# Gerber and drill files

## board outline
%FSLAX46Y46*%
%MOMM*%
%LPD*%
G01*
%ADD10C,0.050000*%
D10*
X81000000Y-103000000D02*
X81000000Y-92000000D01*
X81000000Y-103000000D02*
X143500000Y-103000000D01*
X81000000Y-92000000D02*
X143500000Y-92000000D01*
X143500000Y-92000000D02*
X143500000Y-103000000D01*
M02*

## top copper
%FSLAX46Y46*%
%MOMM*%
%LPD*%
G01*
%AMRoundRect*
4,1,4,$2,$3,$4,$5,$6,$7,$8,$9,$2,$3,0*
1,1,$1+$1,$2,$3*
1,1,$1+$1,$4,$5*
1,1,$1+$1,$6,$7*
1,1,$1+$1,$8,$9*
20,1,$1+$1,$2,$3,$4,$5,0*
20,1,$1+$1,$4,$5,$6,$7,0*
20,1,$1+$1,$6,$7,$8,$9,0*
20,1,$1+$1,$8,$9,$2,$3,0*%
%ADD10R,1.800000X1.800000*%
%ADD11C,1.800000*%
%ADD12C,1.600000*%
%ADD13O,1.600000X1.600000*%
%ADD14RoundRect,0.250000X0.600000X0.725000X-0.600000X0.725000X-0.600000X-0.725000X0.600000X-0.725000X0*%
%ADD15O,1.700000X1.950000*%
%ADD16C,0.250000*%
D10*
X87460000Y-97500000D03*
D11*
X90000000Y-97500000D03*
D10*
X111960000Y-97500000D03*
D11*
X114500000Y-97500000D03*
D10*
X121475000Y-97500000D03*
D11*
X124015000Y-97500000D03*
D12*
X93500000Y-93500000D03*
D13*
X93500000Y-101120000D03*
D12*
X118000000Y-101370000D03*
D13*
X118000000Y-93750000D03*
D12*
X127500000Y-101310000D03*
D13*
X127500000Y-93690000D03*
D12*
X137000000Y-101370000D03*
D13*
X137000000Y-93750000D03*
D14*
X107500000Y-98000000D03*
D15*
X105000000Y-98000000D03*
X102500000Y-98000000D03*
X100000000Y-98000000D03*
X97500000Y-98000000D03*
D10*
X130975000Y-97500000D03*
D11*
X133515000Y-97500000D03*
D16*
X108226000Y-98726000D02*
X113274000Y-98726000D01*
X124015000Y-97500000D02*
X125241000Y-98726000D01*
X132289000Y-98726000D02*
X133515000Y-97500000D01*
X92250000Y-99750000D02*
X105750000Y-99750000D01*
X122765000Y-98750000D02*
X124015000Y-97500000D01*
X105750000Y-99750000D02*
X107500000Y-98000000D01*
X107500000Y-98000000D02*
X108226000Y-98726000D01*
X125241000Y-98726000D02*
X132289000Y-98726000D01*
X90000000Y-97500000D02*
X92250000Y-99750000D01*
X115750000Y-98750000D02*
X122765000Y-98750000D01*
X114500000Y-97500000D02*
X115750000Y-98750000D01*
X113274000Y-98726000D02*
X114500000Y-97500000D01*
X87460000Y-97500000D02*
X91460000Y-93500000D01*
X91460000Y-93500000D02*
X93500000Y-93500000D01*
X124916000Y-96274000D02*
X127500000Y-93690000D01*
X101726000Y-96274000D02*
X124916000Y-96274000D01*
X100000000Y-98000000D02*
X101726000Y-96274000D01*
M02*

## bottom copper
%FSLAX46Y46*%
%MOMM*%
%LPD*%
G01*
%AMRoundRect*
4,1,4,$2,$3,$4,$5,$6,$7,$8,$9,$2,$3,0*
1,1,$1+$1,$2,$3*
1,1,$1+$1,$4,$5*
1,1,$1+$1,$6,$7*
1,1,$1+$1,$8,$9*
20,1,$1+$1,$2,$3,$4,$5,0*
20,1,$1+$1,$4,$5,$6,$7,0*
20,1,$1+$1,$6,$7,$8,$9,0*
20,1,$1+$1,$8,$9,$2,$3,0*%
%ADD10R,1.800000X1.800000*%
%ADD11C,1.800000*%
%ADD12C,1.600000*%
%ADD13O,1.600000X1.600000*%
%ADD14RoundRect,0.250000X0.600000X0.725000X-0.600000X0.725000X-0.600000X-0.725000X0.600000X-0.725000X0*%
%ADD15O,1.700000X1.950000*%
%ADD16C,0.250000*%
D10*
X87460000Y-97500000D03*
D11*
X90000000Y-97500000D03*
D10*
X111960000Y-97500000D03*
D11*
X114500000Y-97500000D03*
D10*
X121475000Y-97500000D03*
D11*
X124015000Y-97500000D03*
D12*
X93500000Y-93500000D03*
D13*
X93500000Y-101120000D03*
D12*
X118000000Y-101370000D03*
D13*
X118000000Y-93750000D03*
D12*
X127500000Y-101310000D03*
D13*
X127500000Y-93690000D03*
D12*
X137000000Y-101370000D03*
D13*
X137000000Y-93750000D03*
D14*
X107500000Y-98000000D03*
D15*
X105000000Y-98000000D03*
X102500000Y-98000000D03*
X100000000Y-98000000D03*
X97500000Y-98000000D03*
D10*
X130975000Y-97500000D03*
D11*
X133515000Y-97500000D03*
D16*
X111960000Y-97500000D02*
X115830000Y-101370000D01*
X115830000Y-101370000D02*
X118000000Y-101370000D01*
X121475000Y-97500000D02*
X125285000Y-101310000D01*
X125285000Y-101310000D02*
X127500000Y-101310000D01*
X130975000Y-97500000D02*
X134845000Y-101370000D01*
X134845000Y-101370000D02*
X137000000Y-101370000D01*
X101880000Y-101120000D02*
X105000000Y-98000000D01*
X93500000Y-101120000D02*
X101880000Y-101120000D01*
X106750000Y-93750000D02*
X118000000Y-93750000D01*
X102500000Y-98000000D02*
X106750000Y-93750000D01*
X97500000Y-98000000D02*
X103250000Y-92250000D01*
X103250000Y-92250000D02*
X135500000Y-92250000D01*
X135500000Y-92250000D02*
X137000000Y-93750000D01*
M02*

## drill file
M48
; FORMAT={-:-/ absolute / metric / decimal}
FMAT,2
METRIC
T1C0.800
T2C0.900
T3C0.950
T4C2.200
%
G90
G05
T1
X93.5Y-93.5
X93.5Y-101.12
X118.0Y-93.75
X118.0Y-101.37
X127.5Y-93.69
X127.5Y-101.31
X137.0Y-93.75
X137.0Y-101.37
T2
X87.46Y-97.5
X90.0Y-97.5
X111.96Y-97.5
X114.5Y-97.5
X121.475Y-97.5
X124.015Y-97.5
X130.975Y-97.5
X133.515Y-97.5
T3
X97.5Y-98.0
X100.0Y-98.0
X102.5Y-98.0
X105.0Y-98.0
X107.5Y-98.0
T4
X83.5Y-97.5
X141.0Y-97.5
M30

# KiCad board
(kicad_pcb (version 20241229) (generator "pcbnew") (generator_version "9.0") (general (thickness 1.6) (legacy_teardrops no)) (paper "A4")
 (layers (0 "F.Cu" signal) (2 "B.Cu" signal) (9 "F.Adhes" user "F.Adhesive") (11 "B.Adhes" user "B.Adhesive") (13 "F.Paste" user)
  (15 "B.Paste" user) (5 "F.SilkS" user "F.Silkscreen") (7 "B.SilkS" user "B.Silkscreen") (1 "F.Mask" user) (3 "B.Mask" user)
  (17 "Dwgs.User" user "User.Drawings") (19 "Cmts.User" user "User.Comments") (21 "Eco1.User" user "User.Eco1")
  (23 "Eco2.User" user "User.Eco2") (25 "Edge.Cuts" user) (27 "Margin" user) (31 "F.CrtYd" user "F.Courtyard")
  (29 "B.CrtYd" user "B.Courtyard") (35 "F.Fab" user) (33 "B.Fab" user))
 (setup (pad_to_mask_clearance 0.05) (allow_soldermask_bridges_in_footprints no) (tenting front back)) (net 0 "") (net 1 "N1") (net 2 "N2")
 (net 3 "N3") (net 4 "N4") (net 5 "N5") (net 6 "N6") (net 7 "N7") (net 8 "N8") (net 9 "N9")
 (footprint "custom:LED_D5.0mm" (layer "F.Cu") (at 87.46 97.5)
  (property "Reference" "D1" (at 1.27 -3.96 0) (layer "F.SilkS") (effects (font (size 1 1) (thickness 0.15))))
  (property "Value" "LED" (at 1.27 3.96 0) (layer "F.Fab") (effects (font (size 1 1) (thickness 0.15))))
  (pad "1" thru_hole rect (at 0 0) (size 1.8 1.8) (drill 0.9) (layers "*.Cu" "*.Mask") (remove_unused_layers no) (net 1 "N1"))
  (pad "2" thru_hole circle (at 2.54 0) (size 1.8 1.8) (drill 0.9) (layers "*.Cu" "*.Mask") (remove_unused_layers no) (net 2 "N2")))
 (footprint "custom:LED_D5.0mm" (layer "F.Cu") (at 111.96 97.5)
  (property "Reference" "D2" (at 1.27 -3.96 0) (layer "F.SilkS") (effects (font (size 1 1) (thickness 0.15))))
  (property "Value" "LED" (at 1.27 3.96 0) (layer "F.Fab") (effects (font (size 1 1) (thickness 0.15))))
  (pad "1" thru_hole rect (at 0 0) (size 1.8 1.8) (drill 0.9) (layers "*.Cu" "*.Mask") (remove_unused_layers no) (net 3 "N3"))
  (pad "2" thru_hole circle (at 2.54 0) (size 1.8 1.8) (drill 0.9) (layers "*.Cu" "*.Mask") (remove_unused_layers no) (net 2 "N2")))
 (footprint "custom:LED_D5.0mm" (layer "F.Cu") (at 121.475 97.5)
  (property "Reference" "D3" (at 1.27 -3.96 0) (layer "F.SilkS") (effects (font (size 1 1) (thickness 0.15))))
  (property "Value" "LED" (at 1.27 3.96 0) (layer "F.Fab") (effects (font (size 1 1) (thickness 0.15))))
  (pad "1" thru_hole rect (at 0 0) (size 1.8 1.8) (drill 0.9) (layers "*.Cu" "*.Mask") (remove_unused_layers no) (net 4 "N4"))
  (pad "2" thru_hole circle (at 2.54 0) (size 1.8 1.8) (drill 0.9) (layers "*.Cu" "*.Mask") (remove_unused_layers no) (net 2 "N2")))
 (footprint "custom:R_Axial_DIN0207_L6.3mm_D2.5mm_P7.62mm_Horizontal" (layer "F.Cu") (at 93.5 93.5 -90)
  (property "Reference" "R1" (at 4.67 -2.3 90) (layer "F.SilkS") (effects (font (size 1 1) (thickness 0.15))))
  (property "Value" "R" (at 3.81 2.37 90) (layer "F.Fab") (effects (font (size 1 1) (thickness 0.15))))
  (pad "1" thru_hole circle (at 0 0 270) (size 1.6 1.6) (drill 0.8) (layers "*.Cu" "*.Mask") (remove_unused_layers no) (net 1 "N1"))
  (pad "2" thru_hole oval (at 7.62 0 270) (size 1.6 1.6) (drill 0.8) (layers "*.Cu" "*.Mask") (remove_unused_layers no) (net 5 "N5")))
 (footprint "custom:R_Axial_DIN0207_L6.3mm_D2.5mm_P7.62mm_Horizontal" (layer "F.Cu") (at 118 101.37 90)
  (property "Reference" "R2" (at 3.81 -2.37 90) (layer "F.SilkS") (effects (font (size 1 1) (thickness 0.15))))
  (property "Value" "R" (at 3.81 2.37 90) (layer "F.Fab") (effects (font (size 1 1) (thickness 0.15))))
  (pad "1" thru_hole circle (at 0 0 90) (size 1.6 1.6) (drill 0.8) (layers "*.Cu" "*.Mask") (remove_unused_layers no) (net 3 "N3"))
  (pad "2" thru_hole oval (at 7.62 0 90) (size 1.6 1.6) (drill 0.8) (layers "*.Cu" "*.Mask") (remove_unused_layers no) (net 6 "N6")))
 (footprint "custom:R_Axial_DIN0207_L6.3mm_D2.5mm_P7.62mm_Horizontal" (layer "F.Cu") (at 127.5 101.31 90)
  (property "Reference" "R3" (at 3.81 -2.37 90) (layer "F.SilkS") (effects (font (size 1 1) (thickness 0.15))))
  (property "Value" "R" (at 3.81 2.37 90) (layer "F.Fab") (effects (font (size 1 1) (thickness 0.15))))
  (pad "1" thru_hole circle (at 0 0 90) (size 1.6 1.6) (drill 0.8) (layers "*.Cu" "*.Mask") (remove_unused_layers no) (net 4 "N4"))
  (pad "2" thru_hole oval (at 7.62 0 90) (size 1.6 1.6) (drill 0.8) (layers "*.Cu" "*.Mask") (remove_unused_layers no) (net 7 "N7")))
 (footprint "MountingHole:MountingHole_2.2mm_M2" (layer "F.Cu") (at 83.5 97.5)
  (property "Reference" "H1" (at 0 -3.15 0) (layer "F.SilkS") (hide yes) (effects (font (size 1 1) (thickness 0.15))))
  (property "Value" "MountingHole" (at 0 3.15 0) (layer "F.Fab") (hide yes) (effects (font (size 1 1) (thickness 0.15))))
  (pad "" np_thru_hole circle (at 0 0) (size 2.2 2.2) (drill 2.2) (layers "*.Cu" "*.Mask")))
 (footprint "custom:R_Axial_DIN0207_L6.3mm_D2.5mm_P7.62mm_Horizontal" (layer "F.Cu") (at 137 101.37 90)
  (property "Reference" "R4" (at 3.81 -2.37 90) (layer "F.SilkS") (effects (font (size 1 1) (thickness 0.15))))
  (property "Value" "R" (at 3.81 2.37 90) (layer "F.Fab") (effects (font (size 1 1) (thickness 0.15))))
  (pad "1" thru_hole circle (at 0 0 90) (size 1.6 1.6) (drill 0.8) (layers "*.Cu" "*.Mask") (remove_unused_layers no) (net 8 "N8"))
  (pad "2" thru_hole oval (at 7.62 0 90) (size 1.6 1.6) (drill 0.8) (layers "*.Cu" "*.Mask") (remove_unused_layers no) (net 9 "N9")))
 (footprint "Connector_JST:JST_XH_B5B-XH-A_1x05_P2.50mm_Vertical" (layer "F.Cu") (at 107.5 98 180)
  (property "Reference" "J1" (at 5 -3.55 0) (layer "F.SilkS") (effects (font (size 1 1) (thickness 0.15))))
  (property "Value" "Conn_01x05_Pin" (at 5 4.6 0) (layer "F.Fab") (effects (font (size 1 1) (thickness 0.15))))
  (pad "1" thru_hole roundrect (at 0 0 180) (size 1.7 1.95) (drill 0.95) (layers "*.Cu" "*.Mask") (remove_unused_layers no)
   (roundrect_rratio 0.147059) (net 2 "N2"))
  (pad "2" thru_hole oval (at 2.5 0 180) (size 1.7 1.95) (drill 0.95) (layers "*.Cu" "*.Mask") (remove_unused_layers no) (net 5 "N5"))
  (pad "3" thru_hole oval (at 5 0 180) (size 1.7 1.95) (drill 0.95) (layers "*.Cu" "*.Mask") (remove_unused_layers no) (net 6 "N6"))
  (pad "4" thru_hole oval (at 7.5 0 180) (size 1.7 1.95) (drill 0.95) (layers "*.Cu" "*.Mask") (remove_unused_layers no) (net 7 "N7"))
  (pad "5" thru_hole oval (at 10 0 180) (size 1.7 1.95) (drill 0.95) (layers "*.Cu" "*.Mask") (remove_unused_layers no) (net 9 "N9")))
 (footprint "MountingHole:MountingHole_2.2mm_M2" (layer "F.Cu") (at 141 97.5)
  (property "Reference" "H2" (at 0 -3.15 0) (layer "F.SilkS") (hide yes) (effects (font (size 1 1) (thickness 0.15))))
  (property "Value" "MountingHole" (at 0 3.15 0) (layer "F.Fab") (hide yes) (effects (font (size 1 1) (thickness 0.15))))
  (pad "" np_thru_hole circle (at 0 0) (size 2.2 2.2) (drill 2.2) (layers "*.Cu" "*.Mask")))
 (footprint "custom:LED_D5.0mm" (layer "F.Cu") (at 130.975 97.5)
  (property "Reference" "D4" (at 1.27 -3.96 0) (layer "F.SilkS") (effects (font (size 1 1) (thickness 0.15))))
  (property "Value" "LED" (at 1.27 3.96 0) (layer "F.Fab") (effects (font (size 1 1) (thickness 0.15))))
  (pad "1" thru_hole rect (at 0 0) (size 1.8 1.8) (drill 0.9) (layers "*.Cu" "*.Mask") (remove_unused_layers no) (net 8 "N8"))
  (pad "2" thru_hole circle (at 2.54 0) (size 1.8 1.8) (drill 0.9) (layers "*.Cu" "*.Mask") (remove_unused_layers no) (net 2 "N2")))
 (gr_line (start 81 103) (end 81 92) (stroke (width 0.05) (type solid)) (layer "Edge.Cuts"))
 (gr_line (start 81 103) (end 143.5 103) (stroke (width 0.05) (type default)) (layer "Edge.Cuts"))
 (gr_line (start 81 92) (end 143.5 92) (stroke (width 0.05) (type default)) (layer "Edge.Cuts"))
 (gr_line (start 143.5 92) (end 143.5 103) (stroke (width 0.05) (type solid)) (layer "Edge.Cuts"))
 (segment (start 108.226 98.726) (end 113.274 98.726) (width 0.25) (layer "F.Cu") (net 2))
 (segment (start 124.015 97.5) (end 125.241 98.726) (width 0.25) (layer "F.Cu") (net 2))
 (segment (start 132.289 98.726) (end 133.515 97.5) (width 0.25) (layer "F.Cu") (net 2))
 (segment (start 92.25 99.75) (end 105.75 99.75) (width 0.25) (layer "F.Cu") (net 2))
 (segment (start 122.765 98.75) (end 124.015 97.5) (width 0.25) (layer "F.Cu") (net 2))
 (segment (start 105.75 99.75) (end 107.5 98) (width 0.25) (layer "F.Cu") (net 2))
 (segment (start 107.5 98) (end 108.226 98.726) (width 0.25) (layer "F.Cu") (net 2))
 (segment (start 125.241 98.726) (end 132.289 98.726) (width 0.25) (layer "F.Cu") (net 2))
 (segment (start 90 97.5) (end 92.25 99.75) (width 0.25) (layer "F.Cu") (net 2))
 (segment (start 115.75 98.75) (end 122.765 98.75) (width 0.25) (layer "F.Cu") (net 2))
 (segment (start 114.5 97.5) (end 115.75 98.75) (width 0.25) (layer "F.Cu") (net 2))
 (segment (start 113.274 98.726) (end 114.5 97.5) (width 0.25) (layer "F.Cu") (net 2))
 (segment (start 87.46 97.5) (end 91.46 93.5) (width 0.25) (layer "F.Cu") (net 1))
 (segment (start 91.46 93.5) (end 93.5 93.5) (width 0.25) (layer "F.Cu") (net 1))
 (segment (start 111.96 97.5) (end 115.83 101.37) (width 0.25) (layer "B.Cu") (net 3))
 (segment (start 115.83 101.37) (end 118 101.37) (width 0.25) (layer "B.Cu") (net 3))
 (segment (start 121.475 97.5) (end 125.285 101.31) (width 0.25) (layer "B.Cu") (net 4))
 (segment (start 125.285 101.31) (end 127.5 101.31) (width 0.25) (layer "B.Cu") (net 4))
 (segment (start 130.975 97.5) (end 134.845 101.37) (width 0.25) (layer "B.Cu") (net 8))
 (segment (start 134.845 101.37) (end 137 101.37) (width 0.25) (layer "B.Cu") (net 8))
 (segment (start 101.88 101.12) (end 105 98) (width 0.25) (layer "B.Cu") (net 5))
 (segment (start 93.5 101.12) (end 101.88 101.12) (width 0.25) (layer "B.Cu") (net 5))
 (segment (start 106.75 93.75) (end 118 93.75) (width 0.25) (layer "B.Cu") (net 6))
 (segment (start 102.5 98) (end 106.75 93.75) (width 0.25) (layer "B.Cu") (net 6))
 (segment (start 124.916 96.274) (end 127.5 93.69) (width 0.25) (layer "F.Cu") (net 7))
 (segment (start 101.726 96.274) (end 124.916 96.274) (width 0.25) (layer "F.Cu") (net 7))
 (segment (start 100 98) (end 101.726 96.274) (width 0.25) (layer "F.Cu") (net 7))
 (segment (start 97.5 98) (end 103.25 92.25) (width 0.25) (layer "B.Cu") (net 9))
 (segment (start 103.25 92.25) (end 135.5 92.25) (width 0.25) (layer "B.Cu") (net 9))
 (segment (start 135.5 92.25) (end 137 93.75) (width 0.25) (layer "B.Cu") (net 9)))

